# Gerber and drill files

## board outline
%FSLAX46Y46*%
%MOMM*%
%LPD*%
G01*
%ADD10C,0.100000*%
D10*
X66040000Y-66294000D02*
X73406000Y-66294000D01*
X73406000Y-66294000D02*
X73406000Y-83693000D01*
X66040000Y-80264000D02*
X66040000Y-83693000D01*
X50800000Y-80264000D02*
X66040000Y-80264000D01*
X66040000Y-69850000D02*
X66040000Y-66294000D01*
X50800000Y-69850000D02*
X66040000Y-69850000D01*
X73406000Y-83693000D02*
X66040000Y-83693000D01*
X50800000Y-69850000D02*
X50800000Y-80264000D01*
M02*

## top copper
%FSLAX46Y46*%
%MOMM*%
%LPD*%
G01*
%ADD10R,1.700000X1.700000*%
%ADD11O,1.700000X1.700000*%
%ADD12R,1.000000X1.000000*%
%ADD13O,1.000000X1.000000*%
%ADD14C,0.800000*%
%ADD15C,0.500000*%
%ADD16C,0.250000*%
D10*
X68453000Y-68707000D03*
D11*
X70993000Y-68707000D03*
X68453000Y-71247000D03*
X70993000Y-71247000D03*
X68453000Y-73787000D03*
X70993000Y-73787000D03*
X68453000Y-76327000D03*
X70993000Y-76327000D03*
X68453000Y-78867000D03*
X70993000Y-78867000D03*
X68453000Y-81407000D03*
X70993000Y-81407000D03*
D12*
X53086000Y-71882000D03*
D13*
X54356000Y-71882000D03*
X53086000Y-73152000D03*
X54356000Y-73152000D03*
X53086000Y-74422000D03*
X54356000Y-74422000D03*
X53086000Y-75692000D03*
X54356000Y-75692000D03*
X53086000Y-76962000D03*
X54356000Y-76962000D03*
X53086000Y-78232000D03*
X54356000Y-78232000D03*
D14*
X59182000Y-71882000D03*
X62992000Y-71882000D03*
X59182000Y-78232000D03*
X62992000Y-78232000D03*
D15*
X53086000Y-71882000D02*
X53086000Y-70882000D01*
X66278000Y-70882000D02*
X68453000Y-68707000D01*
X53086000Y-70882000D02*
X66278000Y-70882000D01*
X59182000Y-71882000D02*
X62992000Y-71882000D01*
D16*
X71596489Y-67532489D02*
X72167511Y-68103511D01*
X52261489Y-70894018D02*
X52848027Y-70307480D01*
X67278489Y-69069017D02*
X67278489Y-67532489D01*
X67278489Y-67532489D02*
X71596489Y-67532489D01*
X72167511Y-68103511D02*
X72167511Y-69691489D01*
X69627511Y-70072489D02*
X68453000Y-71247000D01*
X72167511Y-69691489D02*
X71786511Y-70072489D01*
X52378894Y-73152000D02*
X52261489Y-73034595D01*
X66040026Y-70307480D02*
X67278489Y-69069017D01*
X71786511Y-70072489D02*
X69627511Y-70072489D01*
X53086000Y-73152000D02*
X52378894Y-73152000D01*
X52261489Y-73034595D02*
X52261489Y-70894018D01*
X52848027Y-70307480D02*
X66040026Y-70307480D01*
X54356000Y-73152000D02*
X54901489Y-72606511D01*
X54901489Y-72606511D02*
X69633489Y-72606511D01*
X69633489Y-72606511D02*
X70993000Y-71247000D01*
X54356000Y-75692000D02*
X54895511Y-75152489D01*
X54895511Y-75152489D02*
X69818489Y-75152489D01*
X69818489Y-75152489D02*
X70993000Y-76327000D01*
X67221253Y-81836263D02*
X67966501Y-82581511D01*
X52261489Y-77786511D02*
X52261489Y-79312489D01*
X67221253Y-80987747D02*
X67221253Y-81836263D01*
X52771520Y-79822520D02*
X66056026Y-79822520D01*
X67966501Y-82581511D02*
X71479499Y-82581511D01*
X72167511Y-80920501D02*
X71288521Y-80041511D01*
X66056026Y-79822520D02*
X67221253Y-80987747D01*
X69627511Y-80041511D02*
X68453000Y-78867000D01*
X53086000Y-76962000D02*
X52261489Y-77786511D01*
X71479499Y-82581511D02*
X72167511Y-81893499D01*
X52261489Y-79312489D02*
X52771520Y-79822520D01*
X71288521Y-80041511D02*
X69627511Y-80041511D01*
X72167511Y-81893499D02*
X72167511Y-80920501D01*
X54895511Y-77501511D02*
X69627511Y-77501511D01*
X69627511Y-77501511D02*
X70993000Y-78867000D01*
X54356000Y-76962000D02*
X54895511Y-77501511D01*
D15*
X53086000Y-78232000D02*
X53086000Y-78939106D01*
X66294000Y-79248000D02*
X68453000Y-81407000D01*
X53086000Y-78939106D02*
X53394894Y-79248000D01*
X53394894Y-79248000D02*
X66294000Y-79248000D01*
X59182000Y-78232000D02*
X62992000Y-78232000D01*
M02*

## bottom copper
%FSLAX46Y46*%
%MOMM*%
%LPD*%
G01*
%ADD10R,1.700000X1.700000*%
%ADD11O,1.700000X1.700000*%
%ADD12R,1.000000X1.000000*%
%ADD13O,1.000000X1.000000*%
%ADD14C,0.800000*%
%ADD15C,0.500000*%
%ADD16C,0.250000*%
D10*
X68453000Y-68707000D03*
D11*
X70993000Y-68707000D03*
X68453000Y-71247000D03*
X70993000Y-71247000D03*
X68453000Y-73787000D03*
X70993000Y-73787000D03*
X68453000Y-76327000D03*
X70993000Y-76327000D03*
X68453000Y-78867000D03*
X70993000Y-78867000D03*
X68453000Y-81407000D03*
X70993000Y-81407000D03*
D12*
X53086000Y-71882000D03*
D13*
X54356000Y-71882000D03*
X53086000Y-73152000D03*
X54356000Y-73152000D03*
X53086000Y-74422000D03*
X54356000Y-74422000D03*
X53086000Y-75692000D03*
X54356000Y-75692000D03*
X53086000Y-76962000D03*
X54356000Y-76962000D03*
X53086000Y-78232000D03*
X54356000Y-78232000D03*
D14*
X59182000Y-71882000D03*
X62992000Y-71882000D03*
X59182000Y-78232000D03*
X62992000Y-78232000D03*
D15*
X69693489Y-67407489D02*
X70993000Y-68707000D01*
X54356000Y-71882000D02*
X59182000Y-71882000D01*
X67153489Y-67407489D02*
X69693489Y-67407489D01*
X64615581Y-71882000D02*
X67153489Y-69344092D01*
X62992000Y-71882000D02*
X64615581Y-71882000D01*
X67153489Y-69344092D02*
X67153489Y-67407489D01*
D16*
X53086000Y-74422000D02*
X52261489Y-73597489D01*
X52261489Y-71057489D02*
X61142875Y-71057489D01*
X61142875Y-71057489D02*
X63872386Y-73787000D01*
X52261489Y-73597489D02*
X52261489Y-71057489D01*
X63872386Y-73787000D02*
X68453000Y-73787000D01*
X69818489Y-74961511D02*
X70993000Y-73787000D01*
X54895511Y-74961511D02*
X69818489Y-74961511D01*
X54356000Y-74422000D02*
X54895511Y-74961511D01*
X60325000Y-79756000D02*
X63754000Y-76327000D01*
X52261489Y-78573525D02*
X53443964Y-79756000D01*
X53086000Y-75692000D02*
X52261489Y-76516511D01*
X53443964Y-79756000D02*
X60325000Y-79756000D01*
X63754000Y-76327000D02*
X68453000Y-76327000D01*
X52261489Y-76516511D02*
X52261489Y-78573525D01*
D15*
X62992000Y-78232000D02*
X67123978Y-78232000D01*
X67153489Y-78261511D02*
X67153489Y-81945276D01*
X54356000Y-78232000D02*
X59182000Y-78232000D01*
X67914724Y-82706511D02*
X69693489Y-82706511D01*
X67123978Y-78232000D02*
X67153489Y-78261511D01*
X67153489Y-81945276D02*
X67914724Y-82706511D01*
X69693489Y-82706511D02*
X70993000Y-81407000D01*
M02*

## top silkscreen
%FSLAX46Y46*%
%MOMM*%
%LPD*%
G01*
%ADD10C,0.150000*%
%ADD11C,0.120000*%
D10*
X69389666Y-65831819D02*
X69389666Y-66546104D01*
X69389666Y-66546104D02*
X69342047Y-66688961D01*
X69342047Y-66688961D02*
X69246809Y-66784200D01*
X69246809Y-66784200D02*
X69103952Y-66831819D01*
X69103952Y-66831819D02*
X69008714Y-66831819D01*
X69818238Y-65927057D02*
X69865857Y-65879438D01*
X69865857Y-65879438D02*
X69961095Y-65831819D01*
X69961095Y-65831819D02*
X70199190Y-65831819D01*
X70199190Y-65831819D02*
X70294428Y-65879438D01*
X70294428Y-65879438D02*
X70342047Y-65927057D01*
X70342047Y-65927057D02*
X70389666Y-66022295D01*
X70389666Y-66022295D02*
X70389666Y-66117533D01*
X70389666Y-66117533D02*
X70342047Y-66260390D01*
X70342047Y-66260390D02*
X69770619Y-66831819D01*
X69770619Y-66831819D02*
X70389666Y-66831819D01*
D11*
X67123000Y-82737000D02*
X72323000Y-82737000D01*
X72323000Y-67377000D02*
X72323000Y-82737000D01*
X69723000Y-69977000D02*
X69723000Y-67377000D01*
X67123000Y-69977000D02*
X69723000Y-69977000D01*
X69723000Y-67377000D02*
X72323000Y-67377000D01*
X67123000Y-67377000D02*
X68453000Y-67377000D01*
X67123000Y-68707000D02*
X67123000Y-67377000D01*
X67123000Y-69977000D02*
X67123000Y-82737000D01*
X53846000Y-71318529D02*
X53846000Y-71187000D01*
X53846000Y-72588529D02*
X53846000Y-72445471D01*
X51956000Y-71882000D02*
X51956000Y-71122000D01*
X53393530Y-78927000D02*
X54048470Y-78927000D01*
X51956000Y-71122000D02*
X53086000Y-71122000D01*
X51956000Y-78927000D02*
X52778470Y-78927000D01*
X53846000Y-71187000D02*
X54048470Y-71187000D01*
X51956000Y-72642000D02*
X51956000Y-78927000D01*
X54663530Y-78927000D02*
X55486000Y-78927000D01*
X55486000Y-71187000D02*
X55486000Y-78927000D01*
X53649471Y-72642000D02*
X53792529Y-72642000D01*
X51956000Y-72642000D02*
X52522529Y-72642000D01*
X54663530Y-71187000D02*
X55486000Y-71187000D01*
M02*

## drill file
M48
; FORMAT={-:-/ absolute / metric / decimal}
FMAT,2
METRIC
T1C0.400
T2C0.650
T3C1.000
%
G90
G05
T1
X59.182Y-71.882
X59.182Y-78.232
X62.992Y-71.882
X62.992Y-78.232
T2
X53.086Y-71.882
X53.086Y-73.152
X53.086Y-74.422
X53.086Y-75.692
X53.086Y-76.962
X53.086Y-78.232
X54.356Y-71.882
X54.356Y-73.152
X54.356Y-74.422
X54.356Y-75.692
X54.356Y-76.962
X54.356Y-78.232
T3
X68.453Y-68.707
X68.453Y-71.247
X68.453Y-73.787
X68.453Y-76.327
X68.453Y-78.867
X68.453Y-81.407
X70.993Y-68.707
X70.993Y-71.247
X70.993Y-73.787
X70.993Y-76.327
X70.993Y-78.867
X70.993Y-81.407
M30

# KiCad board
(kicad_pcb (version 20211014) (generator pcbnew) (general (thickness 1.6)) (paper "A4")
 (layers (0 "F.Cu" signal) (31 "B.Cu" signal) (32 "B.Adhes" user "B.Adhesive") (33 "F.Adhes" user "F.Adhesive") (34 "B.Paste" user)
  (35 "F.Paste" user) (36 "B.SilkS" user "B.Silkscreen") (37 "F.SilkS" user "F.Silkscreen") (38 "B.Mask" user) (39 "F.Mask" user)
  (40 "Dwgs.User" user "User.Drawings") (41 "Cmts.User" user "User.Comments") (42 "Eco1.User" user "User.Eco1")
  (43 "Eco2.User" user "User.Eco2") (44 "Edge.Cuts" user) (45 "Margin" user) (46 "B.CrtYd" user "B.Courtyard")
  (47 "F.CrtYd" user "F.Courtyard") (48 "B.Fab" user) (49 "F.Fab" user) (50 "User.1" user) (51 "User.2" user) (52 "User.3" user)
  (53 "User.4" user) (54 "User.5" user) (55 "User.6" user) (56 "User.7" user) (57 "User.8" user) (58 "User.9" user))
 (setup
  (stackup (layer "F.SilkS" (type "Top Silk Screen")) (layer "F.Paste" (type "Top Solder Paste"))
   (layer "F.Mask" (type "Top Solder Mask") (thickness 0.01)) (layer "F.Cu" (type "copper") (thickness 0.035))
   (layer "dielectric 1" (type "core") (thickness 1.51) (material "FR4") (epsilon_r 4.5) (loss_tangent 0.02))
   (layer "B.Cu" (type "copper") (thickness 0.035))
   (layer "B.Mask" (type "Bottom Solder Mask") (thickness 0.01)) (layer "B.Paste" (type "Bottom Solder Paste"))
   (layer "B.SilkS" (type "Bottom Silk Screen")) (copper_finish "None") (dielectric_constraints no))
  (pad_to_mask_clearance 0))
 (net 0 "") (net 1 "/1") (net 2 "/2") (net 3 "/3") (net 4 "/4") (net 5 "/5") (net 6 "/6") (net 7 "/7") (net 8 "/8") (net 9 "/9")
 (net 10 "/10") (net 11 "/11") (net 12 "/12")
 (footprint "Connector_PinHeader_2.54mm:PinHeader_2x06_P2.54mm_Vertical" (layer "F.Cu") (at 68.453 68.707)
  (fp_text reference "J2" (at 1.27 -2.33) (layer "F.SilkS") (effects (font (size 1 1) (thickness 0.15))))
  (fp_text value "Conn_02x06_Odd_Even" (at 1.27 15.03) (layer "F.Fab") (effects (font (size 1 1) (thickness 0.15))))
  (fp_line (start -1.33 14.03) (end 3.87 14.03) (layer "F.SilkS") (width 0.12))
  (fp_line (start 3.87 -1.33) (end 3.87 14.03) (layer "F.SilkS") (width 0.12))
  (fp_line (start 1.27 1.27) (end 1.27 -1.33) (layer "F.SilkS") (width 0.12))
  (fp_line (start -1.33 1.27) (end 1.27 1.27) (layer "F.SilkS") (width 0.12))
  (fp_line (start 1.27 -1.33) (end 3.87 -1.33) (layer "F.SilkS") (width 0.12))
  (fp_line (start -1.33 -1.33) (end 0 -1.33) (layer "F.SilkS") (width 0.12))
  (fp_line (start -1.33 0) (end -1.33 -1.33) (layer "F.SilkS") (width 0.12))
  (fp_line (start -1.33 1.27) (end -1.33 14.03) (layer "F.SilkS") (width 0.12))
  (pad "1" thru_hole rect (at 0 0) (size 1.7 1.7) (drill 1) (layers *.Cu *.Mask) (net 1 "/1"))
  (pad "2" thru_hole oval (at 2.54 0) (size 1.7 1.7) (drill 1) (layers *.Cu *.Mask) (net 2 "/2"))
  (pad "3" thru_hole oval (at 0 2.54) (size 1.7 1.7) (drill 1) (layers *.Cu *.Mask) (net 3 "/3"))
  (pad "4" thru_hole oval (at 2.54 2.54) (size 1.7 1.7) (drill 1) (layers *.Cu *.Mask) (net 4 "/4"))
  (pad "5" thru_hole oval (at 0 5.08) (size 1.7 1.7) (drill 1) (layers *.Cu *.Mask) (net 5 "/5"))
  (pad "6" thru_hole oval (at 2.54 5.08) (size 1.7 1.7) (drill 1) (layers *.Cu *.Mask) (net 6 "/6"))
  (pad "7" thru_hole oval (at 0 7.62) (size 1.7 1.7) (drill 1) (layers *.Cu *.Mask) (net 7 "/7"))
  (pad "8" thru_hole oval (at 2.54 7.62) (size 1.7 1.7) (drill 1) (layers *.Cu *.Mask) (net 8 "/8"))
  (pad "9" thru_hole oval (at 0 10.16) (size 1.7 1.7) (drill 1) (layers *.Cu *.Mask) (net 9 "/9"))
  (pad "10" thru_hole oval (at 2.54 10.16) (size 1.7 1.7) (drill 1) (layers *.Cu *.Mask) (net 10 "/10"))
  (pad "11" thru_hole oval (at 0 12.7) (size 1.7 1.7) (drill 1) (layers *.Cu *.Mask) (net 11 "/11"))
  (pad "12" thru_hole oval (at 2.54 12.7) (size 1.7 1.7) (drill 1) (layers *.Cu *.Mask) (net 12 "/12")))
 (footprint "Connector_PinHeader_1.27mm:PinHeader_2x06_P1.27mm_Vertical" (layer "F.Cu") (at 53.086 71.882)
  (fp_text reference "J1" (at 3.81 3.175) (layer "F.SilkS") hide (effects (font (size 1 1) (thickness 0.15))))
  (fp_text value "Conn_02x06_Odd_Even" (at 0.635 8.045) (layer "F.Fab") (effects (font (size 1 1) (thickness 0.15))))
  (fp_line (start 0.76 -0.563471) (end 0.76 -0.695) (layer "F.SilkS") (width 0.12))
  (fp_line (start 0.76 0.706529) (end 0.76 0.563471) (layer "F.SilkS") (width 0.12))
  (fp_line (start -1.13 0) (end -1.13 -0.76) (layer "F.SilkS") (width 0.12))
  (fp_line (start 0.30753 7.045) (end 0.96247 7.045) (layer "F.SilkS") (width 0.12))
  (fp_line (start -1.13 -0.76) (end 0 -0.76) (layer "F.SilkS") (width 0.12))
  (fp_line (start -1.13 7.045) (end -0.30753 7.045) (layer "F.SilkS") (width 0.12))
  (fp_line (start 0.76 -0.695) (end 0.96247 -0.695) (layer "F.SilkS") (width 0.12))
  (fp_line (start -1.13 0.76) (end -1.13 7.045) (layer "F.SilkS") (width 0.12))
  (fp_line (start 1.57753 7.045) (end 2.4 7.045) (layer "F.SilkS") (width 0.12))
  (fp_line (start 2.4 -0.695) (end 2.4 7.045) (layer "F.SilkS") (width 0.12))
  (fp_line (start 0.563471 0.76) (end 0.706529 0.76) (layer "F.SilkS") (width 0.12))
  (fp_line (start -1.13 0.76) (end -0.563471 0.76) (layer "F.SilkS") (width 0.12))
  (fp_line (start 1.57753 -0.695) (end 2.4 -0.695) (layer "F.SilkS") (width 0.12))
  (pad "1" thru_hole rect (at 0 0) (size 1 1) (drill 0.65) (layers *.Cu *.Mask) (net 1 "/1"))
  (pad "2" thru_hole oval (at 1.27 0) (size 1 1) (drill 0.65) (layers *.Cu *.Mask) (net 2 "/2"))
  (pad "3" thru_hole oval (at 0 1.27) (size 1 1) (drill 0.65) (layers *.Cu *.Mask) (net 3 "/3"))
  (pad "4" thru_hole oval (at 1.27 1.27) (size 1 1) (drill 0.65) (layers *.Cu *.Mask) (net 4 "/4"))
  (pad "5" thru_hole oval (at 0 2.54) (size 1 1) (drill 0.65) (layers *.Cu *.Mask) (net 5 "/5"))
  (pad "6" thru_hole oval (at 1.27 2.54) (size 1 1) (drill 0.65) (layers *.Cu *.Mask) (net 6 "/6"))
  (pad "7" thru_hole oval (at 0 3.81) (size 1 1) (drill 0.65) (layers *.Cu *.Mask) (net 7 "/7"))
  (pad "8" thru_hole oval (at 1.27 3.81) (size 1 1) (drill 0.65) (layers *.Cu *.Mask) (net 8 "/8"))
  (pad "9" thru_hole oval (at 0 5.08) (size 1 1) (drill 0.65) (layers *.Cu *.Mask) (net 9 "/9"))
  (pad "10" thru_hole oval (at 1.27 5.08) (size 1 1) (drill 0.65) (layers *.Cu *.Mask) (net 10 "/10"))
  (pad "11" thru_hole oval (at 0 6.35) (size 1 1) (drill 0.65) (layers *.Cu *.Mask) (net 11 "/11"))
  (pad "12" thru_hole oval (at 1.27 6.35) (size 1 1) (drill 0.65) (layers *.Cu *.Mask) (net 12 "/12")))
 (gr_line (start 66.04 66.294) (end 73.406 66.294) (layer "Edge.Cuts") (width 0.1))
 (gr_line (start 73.406 66.294) (end 73.406 83.693) (layer "Edge.Cuts") (width 0.1))
 (gr_line (start 66.04 80.264) (end 66.04 83.693) (layer "Edge.Cuts") (width 0.1))
 (gr_line (start 50.8 80.264) (end 66.04 80.264) (layer "Edge.Cuts") (width 0.1))
 (gr_line (start 66.04 69.85) (end 66.04 66.294) (layer "Edge.Cuts") (width 0.1))
 (gr_line (start 50.8 69.85) (end 66.04 69.85) (layer "Edge.Cuts") (width 0.1))
 (gr_line (start 73.406 83.693) (end 66.04 83.693) (layer "Edge.Cuts") (width 0.1))
 (gr_line (start 50.8 69.85) (end 50.8 80.264) (layer "Edge.Cuts") (width 0.1))
 (segment (start 53.086 71.882) (end 53.086 70.882) (width 0.5) (layer "F.Cu") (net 1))
 (segment (start 66.278 70.882) (end 68.453 68.707) (width 0.5) (layer "F.Cu") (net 1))
 (segment (start 53.086 70.882) (end 66.278 70.882) (width 0.5) (layer "F.Cu") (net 1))
 (segment (start 59.182 71.882) (end 62.992 71.882) (width 0.5) (layer "F.Cu") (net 2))
 (via (at 59.182 71.882) (size 0.8) (drill 0.4) (layers "F.Cu" "B.Cu") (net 2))
 (via (at 62.992 71.882) (size 0.8) (drill 0.4) (layers "F.Cu" "B.Cu") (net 2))
 (segment (start 69.693489 67.407489) (end 70.993 68.707) (width 0.5) (layer "B.Cu") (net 2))
 (segment (start 54.356 71.882) (end 59.182 71.882) (width 0.5) (layer "B.Cu") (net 2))
 (segment (start 67.153489 67.407489) (end 69.693489 67.407489) (width 0.5) (layer "B.Cu") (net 2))
 (segment (start 64.615581 71.882) (end 67.153489 69.344092) (width 0.5) (layer "B.Cu") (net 2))
 (segment (start 62.992 71.882) (end 64.615581 71.882) (width 0.5) (layer "B.Cu") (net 2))
 (segment (start 67.153489 69.344092) (end 67.153489 67.407489) (width 0.5) (layer "B.Cu") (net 2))
 (segment (start 71.596489 67.532489) (end 72.167511 68.103511) (width 0.25) (layer "F.Cu") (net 3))
 (segment (start 52.261489 70.894018) (end 52.848027 70.30748) (width 0.25) (layer "F.Cu") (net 3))
 (segment (start 67.278489 69.069017) (end 67.278489 67.532489) (width 0.25) (layer "F.Cu") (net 3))
 (segment (start 67.278489 67.532489) (end 71.596489 67.532489) (width 0.25) (layer "F.Cu") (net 3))
 (segment (start 72.167511 68.103511) (end 72.167511 69.691489) (width 0.25) (layer "F.Cu") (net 3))
 (segment (start 69.627511 70.072489) (end 68.453 71.247) (width 0.25) (layer "F.Cu") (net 3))
 (segment (start 72.167511 69.691489) (end 71.786511 70.072489) (width 0.25) (layer "F.Cu") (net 3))
 (segment (start 52.378894 73.152) (end 52.261489 73.034595) (width 0.25) (layer "F.Cu") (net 3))
 (segment (start 66.040026 70.30748) (end 67.278489 69.069017) (width 0.25) (layer "F.Cu") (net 3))
 (segment (start 71.786511 70.072489) (end 69.627511 70.072489) (width 0.25) (layer "F.Cu") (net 3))
 (segment (start 53.086 73.152) (end 52.378894 73.152) (width 0.25) (layer "F.Cu") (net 3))
 (segment (start 52.261489 73.034595) (end 52.261489 70.894018) (width 0.25) (layer "F.Cu") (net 3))
 (segment (start 52.848027 70.30748) (end 66.040026 70.30748) (width 0.25) (layer "F.Cu") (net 3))
 (segment (start 54.356 73.152) (end 54.901489 72.606511) (width 0.25) (layer "F.Cu") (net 4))
 (segment (start 54.901489 72.606511) (end 69.633489 72.606511) (width 0.25) (layer "F.Cu") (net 4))
 (segment (start 69.633489 72.606511) (end 70.993 71.247) (width 0.25) (layer "F.Cu") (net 4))
 (segment (start 53.086 74.422) (end 52.261489 73.597489) (width 0.25) (layer "B.Cu") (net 5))
 (segment (start 52.261489 71.057489) (end 61.142875 71.057489) (width 0.25) (layer "B.Cu") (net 5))
 (segment (start 61.142875 71.057489) (end 63.872386 73.787) (width 0.25) (layer "B.Cu") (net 5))
 (segment (start 52.261489 73.597489) (end 52.261489 71.057489) (width 0.25) (layer "B.Cu") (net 5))
 (segment (start 63.872386 73.787) (end 68.453 73.787) (width 0.25) (layer "B.Cu") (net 5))
 (segment (start 69.818489 74.961511) (end 70.993 73.787) (width 0.25) (layer "B.Cu") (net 6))
 (segment (start 54.895511 74.961511) (end 69.818489 74.961511) (width 0.25) (layer "B.Cu") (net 6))
 (segment (start 54.356 74.422) (end 54.895511 74.961511) (width 0.25) (layer "B.Cu") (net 6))
 (segment (start 60.325 79.756) (end 63.754 76.327) (width 0.25) (layer "B.Cu") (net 7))
 (segment (start 52.261489 78.573525) (end 53.443964 79.756) (width 0.25) (layer "B.Cu") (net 7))
 (segment (start 53.086 75.692) (end 52.261489 76.516511) (width 0.25) (layer "B.Cu") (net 7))
 (segment (start 53.443964 79.756) (end 60.325 79.756) (width 0.25) (layer "B.Cu") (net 7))
 (segment (start 63.754 76.327) (end 68.453 76.327) (width 0.25) (layer "B.Cu") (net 7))
 (segment (start 52.261489 76.516511) (end 52.261489 78.573525) (width 0.25) (layer "B.Cu") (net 7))
 (segment (start 54.356 75.692) (end 54.895511 75.152489) (width 0.25) (layer "F.Cu") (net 8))
 (segment (start 54.895511 75.152489) (end 69.818489 75.152489) (width 0.25) (layer "F.Cu") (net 8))
 (segment (start 69.818489 75.152489) (end 70.993 76.327) (width 0.25) (layer "F.Cu") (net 8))
 (segment (start 67.221253 81.836263) (end 67.966501 82.581511) (width 0.25) (layer "F.Cu") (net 9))
 (segment (start 52.261489 77.786511) (end 52.261489 79.312489) (width 0.25) (layer "F.Cu") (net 9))
 (segment (start 67.221253 80.987747) (end 67.221253 81.836263) (width 0.25) (layer "F.Cu") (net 9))
 (segment (start 52.77152 79.82252) (end 66.056026 79.82252) (width 0.25) (layer "F.Cu") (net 9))
 (segment (start 67.966501 82.581511) (end 71.479499 82.581511) (width 0.25) (layer "F.Cu") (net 9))
 (segment (start 72.167511 80.920501) (end 71.288521 80.041511) (width 0.25) (layer "F.Cu") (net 9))
 (segment (start 66.056026 79.82252) (end 67.221253 80.987747) (width 0.25) (layer "F.Cu") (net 9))
 (segment (start 69.627511 80.041511) (end 68.453 78.867) (width 0.25) (layer "F.Cu") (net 9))
 (segment (start 53.086 76.962) (end 52.261489 77.786511) (width 0.25) (layer "F.Cu") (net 9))
 (segment (start 71.479499 82.581511) (end 72.167511 81.893499) (width 0.25) (layer "F.Cu") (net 9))
 (segment (start 52.261489 79.312489) (end 52.77152 79.82252) (width 0.25) (layer "F.Cu") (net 9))
 (segment (start 71.288521 80.041511) (end 69.627511 80.041511) (width 0.25) (layer "F.Cu") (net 9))
 (segment (start 72.167511 81.893499) (end 72.167511 80.920501) (width 0.25) (layer "F.Cu") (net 9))
 (segment (start 54.895511 77.501511) (end 69.627511 77.501511) (width 0.25) (layer "F.Cu") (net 10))
 (segment (start 69.627511 77.501511) (end 70.993 78.867) (width 0.25) (layer "F.Cu") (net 10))
 (segment (start 54.356 76.962) (end 54.895511 77.501511) (width 0.25) (layer "F.Cu") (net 10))
 (segment (start 53.086 78.232) (end 53.086 78.939106) (width 0.5) (layer "F.Cu") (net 11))
 (segment (start 66.294 79.248) (end 68.453 81.407) (width 0.5) (layer "F.Cu") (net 11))
 (segment (start 53.086 78.939106) (end 53.394894 79.248) (width 0.5) (layer "F.Cu") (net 11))
 (segment (start 53.394894 79.248) (end 66.294 79.248) (width 0.5) (layer "F.Cu") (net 11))
 (segment (start 59.182 78.232) (end 62.992 78.232) (width 0.5) (layer "F.Cu") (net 12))
 (via (at 59.182 78.232) (size 0.8) (drill 0.4) (layers "F.Cu" "B.Cu") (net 12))
 (via (at 62.992 78.232) (size 0.8) (drill 0.4) (layers "F.Cu" "B.Cu") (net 12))
 (segment (start 62.992 78.232) (end 67.123978 78.232) (width 0.5) (layer "B.Cu") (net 12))
 (segment (start 67.153489 78.261511) (end 67.153489 81.945276) (width 0.5) (layer "B.Cu") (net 12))
 (segment (start 54.356 78.232) (end 59.182 78.232) (width 0.5) (layer "B.Cu") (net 12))
 (segment (start 67.914724 82.706511) (end 69.693489 82.706511) (width 0.5) (layer "B.Cu") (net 12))
 (segment (start 67.123978 78.232) (end 67.153489 78.261511) (width 0.5) (layer "B.Cu") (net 12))
 (segment (start 67.153489 81.945276) (end 67.914724 82.706511) (width 0.5) (layer "B.Cu") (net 12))
 (segment (start 69.693489 82.706511) (end 70.993 81.407) (width 0.5) (layer "B.Cu") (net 12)))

